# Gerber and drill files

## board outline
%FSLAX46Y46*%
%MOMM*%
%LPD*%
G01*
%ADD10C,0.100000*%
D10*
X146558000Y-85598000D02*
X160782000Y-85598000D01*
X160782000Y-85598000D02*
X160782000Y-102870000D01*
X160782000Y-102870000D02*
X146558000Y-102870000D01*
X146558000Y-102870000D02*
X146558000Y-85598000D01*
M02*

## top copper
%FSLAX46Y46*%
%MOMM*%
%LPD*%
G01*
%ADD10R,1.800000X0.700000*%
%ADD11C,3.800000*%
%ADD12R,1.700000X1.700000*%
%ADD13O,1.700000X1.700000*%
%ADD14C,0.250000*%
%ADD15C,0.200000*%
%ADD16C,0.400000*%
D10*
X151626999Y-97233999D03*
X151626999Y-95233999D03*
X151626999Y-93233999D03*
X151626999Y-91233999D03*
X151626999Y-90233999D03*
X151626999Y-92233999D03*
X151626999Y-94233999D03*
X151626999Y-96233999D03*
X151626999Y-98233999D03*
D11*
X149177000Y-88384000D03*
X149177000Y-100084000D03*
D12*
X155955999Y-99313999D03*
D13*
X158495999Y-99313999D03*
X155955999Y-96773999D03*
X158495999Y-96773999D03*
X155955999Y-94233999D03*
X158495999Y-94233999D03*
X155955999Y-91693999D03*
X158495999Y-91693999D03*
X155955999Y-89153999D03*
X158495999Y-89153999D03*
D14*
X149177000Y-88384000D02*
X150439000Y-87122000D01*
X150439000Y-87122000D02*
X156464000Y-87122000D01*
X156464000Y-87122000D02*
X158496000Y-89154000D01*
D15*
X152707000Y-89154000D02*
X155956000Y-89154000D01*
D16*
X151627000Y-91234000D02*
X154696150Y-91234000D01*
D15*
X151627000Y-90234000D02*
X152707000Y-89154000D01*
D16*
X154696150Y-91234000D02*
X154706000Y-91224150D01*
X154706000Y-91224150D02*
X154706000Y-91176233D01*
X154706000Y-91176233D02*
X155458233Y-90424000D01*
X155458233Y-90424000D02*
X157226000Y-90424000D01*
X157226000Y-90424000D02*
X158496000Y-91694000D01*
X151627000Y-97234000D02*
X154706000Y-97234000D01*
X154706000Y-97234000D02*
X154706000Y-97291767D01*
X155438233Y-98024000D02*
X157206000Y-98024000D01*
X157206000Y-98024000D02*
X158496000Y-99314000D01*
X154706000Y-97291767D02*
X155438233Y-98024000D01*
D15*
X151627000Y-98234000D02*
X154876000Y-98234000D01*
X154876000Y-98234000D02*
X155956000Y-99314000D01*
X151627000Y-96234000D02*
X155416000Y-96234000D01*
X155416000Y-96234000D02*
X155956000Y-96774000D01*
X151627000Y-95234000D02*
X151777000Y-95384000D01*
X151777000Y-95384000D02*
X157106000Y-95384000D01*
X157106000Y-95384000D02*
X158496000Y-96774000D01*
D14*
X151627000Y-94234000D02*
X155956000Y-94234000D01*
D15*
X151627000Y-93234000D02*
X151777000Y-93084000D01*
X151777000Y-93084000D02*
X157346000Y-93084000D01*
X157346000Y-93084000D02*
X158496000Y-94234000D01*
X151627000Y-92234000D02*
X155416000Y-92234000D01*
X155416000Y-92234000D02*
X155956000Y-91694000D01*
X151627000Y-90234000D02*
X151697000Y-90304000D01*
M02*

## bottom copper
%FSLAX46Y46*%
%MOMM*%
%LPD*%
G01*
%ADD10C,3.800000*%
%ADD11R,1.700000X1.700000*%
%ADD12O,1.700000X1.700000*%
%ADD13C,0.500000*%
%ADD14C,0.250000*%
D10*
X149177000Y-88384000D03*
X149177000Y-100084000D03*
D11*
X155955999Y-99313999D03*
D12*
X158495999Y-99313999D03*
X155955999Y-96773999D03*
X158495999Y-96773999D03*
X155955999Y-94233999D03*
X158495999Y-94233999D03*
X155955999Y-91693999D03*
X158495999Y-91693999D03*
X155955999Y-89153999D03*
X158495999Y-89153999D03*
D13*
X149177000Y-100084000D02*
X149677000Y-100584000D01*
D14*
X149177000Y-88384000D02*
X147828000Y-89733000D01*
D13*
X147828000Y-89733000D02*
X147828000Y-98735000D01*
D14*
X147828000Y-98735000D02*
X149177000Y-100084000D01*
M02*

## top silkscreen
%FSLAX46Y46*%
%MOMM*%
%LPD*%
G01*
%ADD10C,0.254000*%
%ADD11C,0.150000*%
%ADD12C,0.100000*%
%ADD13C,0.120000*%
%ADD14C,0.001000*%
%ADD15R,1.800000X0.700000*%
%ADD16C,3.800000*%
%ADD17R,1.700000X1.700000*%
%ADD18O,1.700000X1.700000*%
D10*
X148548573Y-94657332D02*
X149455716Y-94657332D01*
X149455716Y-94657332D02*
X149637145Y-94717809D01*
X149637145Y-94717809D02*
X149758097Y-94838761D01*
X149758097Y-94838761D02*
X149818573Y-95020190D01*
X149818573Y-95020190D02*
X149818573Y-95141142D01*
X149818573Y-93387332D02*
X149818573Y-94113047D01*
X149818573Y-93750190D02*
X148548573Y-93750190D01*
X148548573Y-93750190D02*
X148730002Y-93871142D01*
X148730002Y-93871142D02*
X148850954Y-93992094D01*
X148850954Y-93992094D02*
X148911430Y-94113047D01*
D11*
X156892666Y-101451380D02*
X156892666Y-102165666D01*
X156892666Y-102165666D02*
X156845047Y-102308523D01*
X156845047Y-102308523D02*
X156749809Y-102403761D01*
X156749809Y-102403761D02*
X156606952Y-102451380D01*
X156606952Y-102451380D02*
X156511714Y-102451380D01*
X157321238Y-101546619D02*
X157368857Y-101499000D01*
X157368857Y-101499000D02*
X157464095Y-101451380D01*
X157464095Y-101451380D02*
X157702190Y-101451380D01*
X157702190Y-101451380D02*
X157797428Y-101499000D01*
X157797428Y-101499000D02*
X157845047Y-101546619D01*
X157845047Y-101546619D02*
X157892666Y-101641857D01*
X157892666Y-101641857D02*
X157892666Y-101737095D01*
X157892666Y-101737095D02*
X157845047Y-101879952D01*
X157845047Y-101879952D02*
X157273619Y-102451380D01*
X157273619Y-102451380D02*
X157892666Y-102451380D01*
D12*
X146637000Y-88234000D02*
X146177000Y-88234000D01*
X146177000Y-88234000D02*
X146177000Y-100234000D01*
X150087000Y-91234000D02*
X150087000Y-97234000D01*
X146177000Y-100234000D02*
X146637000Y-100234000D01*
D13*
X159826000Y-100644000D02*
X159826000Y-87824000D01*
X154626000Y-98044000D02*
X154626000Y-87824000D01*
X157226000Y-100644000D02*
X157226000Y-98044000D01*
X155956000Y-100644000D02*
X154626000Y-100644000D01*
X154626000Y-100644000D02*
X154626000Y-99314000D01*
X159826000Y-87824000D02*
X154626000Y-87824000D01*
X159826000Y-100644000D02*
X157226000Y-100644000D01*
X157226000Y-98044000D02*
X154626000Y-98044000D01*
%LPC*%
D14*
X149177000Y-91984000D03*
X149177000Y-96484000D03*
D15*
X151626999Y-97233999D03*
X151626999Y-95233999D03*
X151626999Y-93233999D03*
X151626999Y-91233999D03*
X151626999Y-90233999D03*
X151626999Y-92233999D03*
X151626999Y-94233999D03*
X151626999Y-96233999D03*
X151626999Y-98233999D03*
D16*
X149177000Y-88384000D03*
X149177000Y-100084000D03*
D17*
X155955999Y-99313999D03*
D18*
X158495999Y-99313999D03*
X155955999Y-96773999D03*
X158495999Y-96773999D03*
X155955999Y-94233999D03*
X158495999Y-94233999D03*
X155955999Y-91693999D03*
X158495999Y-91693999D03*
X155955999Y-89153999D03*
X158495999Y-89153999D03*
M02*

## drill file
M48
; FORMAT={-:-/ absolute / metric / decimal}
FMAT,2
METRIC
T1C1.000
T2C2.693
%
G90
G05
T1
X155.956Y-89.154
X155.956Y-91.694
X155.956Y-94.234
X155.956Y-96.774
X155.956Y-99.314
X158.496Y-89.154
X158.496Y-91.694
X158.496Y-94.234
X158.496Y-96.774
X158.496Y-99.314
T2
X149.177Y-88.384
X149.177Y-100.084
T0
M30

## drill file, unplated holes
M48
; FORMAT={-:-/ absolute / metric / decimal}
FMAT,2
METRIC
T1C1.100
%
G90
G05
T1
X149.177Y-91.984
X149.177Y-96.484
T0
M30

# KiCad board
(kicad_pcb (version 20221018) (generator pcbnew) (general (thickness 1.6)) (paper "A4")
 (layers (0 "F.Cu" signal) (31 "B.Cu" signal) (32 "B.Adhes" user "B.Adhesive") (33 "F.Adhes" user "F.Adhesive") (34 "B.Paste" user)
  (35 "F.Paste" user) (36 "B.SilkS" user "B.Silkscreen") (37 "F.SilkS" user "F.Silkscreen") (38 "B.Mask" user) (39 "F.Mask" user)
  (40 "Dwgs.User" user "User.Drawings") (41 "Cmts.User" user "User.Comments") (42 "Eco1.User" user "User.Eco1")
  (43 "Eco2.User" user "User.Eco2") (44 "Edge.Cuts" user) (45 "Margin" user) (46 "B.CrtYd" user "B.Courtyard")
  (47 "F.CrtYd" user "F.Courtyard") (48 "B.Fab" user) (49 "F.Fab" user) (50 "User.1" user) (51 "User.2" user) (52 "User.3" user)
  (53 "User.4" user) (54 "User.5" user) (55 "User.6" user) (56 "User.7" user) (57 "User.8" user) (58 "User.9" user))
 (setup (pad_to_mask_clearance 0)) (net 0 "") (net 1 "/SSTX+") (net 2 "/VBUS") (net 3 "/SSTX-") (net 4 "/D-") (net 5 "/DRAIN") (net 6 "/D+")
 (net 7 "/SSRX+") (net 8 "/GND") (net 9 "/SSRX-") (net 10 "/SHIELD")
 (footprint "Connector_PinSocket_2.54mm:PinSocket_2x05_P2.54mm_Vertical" (layer "F.Cu") (at 155.956 99.314 180)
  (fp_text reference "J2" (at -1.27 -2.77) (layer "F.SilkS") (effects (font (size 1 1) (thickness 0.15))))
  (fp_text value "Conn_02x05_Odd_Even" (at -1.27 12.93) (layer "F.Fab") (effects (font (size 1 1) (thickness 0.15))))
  (fp_line (start -3.87 -1.33) (end -3.87 11.49) (stroke (width 0.12) (type solid)) (layer "F.SilkS"))
  (fp_line (start -3.87 -1.33) (end -1.27 -1.33) (stroke (width 0.12) (type solid)) (layer "F.SilkS"))
  (fp_line (start -3.87 11.49) (end 1.33 11.49) (stroke (width 0.12) (type solid)) (layer "F.SilkS"))
  (fp_line (start -1.27 -1.33) (end -1.27 1.27) (stroke (width 0.12) (type solid)) (layer "F.SilkS"))
  (fp_line (start -1.27 1.27) (end 1.33 1.27) (stroke (width 0.12) (type solid)) (layer "F.SilkS"))
  (fp_line (start 0 -1.33) (end 1.33 -1.33) (stroke (width 0.12) (type solid)) (layer "F.SilkS"))
  (fp_line (start 1.33 -1.33) (end 1.33 0) (stroke (width 0.12) (type solid)) (layer "F.SilkS"))
  (fp_line (start 1.33 1.27) (end 1.33 11.49) (stroke (width 0.12) (type solid)) (layer "F.SilkS"))
  (pad "1" thru_hole rect (at 0 0 180) (size 1.7 1.7) (drill 1) (layers "*.Cu" "*.Mask") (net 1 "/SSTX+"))
  (pad "2" thru_hole oval (at -2.54 0 180) (size 1.7 1.7) (drill 1) (layers "*.Cu" "*.Mask") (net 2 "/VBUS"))
  (pad "3" thru_hole oval (at 0 2.54 180) (size 1.7 1.7) (drill 1) (layers "*.Cu" "*.Mask") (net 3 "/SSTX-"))
  (pad "4" thru_hole oval (at -2.54 2.54 180) (size 1.7 1.7) (drill 1) (layers "*.Cu" "*.Mask") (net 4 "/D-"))
  (pad "5" thru_hole oval (at 0 5.08 180) (size 1.7 1.7) (drill 1) (layers "*.Cu" "*.Mask") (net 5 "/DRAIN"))
  (pad "6" thru_hole oval (at -2.54 5.08 180) (size 1.7 1.7) (drill 1) (layers "*.Cu" "*.Mask") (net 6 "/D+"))
  (pad "7" thru_hole oval (at 0 7.62 180) (size 1.7 1.7) (drill 1) (layers "*.Cu" "*.Mask") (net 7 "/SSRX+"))
  (pad "8" thru_hole oval (at -2.54 7.62 180) (size 1.7 1.7) (drill 1) (layers "*.Cu" "*.Mask") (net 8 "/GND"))
  (pad "9" thru_hole oval (at 0 10.16 180) (size 1.7 1.7) (drill 1) (layers "*.Cu" "*.Mask") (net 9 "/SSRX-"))
  (pad "10" thru_hole oval (at -2.54 10.16 180) (size 1.7 1.7) (drill 1) (layers "*.Cu" "*.Mask") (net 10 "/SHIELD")))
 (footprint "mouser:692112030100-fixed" (layer "F.Cu") (at 149.352 94.234 -90)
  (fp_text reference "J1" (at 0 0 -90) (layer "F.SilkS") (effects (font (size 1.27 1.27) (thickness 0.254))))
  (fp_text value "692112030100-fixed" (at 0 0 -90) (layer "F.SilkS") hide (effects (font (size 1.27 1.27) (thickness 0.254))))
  (fp_line (start -6 2.715) (end -6 3.175) (stroke (width 0.1) (type solid)) (layer "F.SilkS"))
  (fp_line (start -6 3.175) (end 6 3.175) (stroke (width 0.1) (type solid)) (layer "F.SilkS"))
  (fp_line (start -3 -0.735) (end 3 -0.735) (stroke (width 0.1) (type solid)) (layer "F.SilkS"))
  (fp_line (start 6 3.175) (end 6 2.715) (stroke (width 0.1) (type solid)) (layer "F.SilkS"))
  (pad "" np_thru_hole circle (at -2.25 0.175 270) (size 0.001 0.001) (drill 1.1) (layers "*.Cu" "*.Mask"))
  (pad "" np_thru_hole circle (at 2.25 0.175 270) (size 0.001 0.001) (drill 1.1) (layers "*.Cu" "*.Mask"))
  (pad "1" smd rect (at 3 -2.275 270) (size 0.7 1.8) (layers "F.Cu" "F.Paste" "F.Mask") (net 2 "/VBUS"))
  (pad "2" smd rect (at 1 -2.275 270) (size 0.7 1.8) (layers "F.Cu" "F.Paste" "F.Mask") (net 4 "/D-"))
  (pad "3" smd rect (at -1 -2.275 270) (size 0.7 1.8) (layers "F.Cu" "F.Paste" "F.Mask") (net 6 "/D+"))
  (pad "4" smd rect (at -3 -2.275 270) (size 0.7 1.8) (layers "F.Cu" "F.Paste" "F.Mask") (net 8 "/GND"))
  (pad "5" smd rect (at -4 -2.275 270) (size 0.7 1.8) (layers "F.Cu" "F.Paste" "F.Mask") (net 9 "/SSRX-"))
  (pad "6" smd rect (at -2 -2.275 270) (size 0.7 1.8) (layers "F.Cu" "F.Paste" "F.Mask") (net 7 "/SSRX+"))
  (pad "7" smd rect (at 0 -2.275 270) (size 0.7 1.8) (layers "F.Cu" "F.Paste" "F.Mask") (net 5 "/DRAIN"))
  (pad "8" smd rect (at 2 -2.275 270) (size 0.7 1.8) (layers "F.Cu" "F.Paste" "F.Mask") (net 3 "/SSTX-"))
  (pad "9" smd rect (at 4 -2.275 270) (size 0.7 1.8) (layers "F.Cu" "F.Paste" "F.Mask") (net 1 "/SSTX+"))
  (pad "10" thru_hole circle (at -5.85 0.175 270) (size 3.8 3.8) (drill 2.6926) (layers "*.Cu" "*.Mask") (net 10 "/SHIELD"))
  (pad "11" thru_hole circle (at 5.85 0.175 270) (size 3.8 3.8) (drill 2.6926) (layers "*.Cu" "*.Mask") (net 10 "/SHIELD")))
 (gr_rect (start 146.558 85.598) (end 160.782 102.87) (stroke (width 0.1) (type solid)) (fill none) (layer "Edge.Cuts"))
 (segment (start 155.438233 98.024) (end 157.206 98.024) (width 0.4) (layer "F.Cu") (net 2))
 (segment (start 154.706 97.291767) (end 155.438233 98.024) (width 0.4) (layer "F.Cu") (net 2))
 (segment (start 154.706 97.234) (end 154.706 97.291767) (width 0.4) (layer "F.Cu") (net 2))
 (segment (start 151.627 97.234) (end 154.706 97.234) (width 0.4) (layer "F.Cu") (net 2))
 (segment (start 157.206 98.024) (end 158.496 99.314) (width 0.4) (layer "F.Cu") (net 2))
 (segment (start 157.106 95.384) (end 158.496 96.774) (width 0.2) (layer "F.Cu") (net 4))
 (segment (start 151.627 95.234) (end 151.777 95.384) (width 0.2) (layer "F.Cu") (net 4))
 (segment (start 151.777 95.384) (end 157.106 95.384) (width 0.2) (layer "F.Cu") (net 4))
 (segment (start 151.777 93.084) (end 157.346 93.084) (width 0.2) (layer "F.Cu") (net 6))
 (segment (start 157.346 93.084) (end 158.496 94.234) (width 0.2) (layer "F.Cu") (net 6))
 (segment (start 151.627 93.234) (end 151.777 93.084) (width 0.2) (layer "F.Cu") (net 6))
 (segment (start 154.69615 91.234) (end 154.706 91.22415) (width 0.4) (layer "F.Cu") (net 8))
 (segment (start 154.706 91.176233) (end 155.458233 90.424) (width 0.4) (layer "F.Cu") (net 8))
 (segment (start 154.706 91.22415) (end 154.706 91.176233) (width 0.4) (layer "F.Cu") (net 8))
 (segment (start 157.226 90.424) (end 158.496 91.694) (width 0.4) (layer "F.Cu") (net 8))
 (segment (start 151.627 91.234) (end 154.69615 91.234) (width 0.4) (layer "F.Cu") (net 8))
 (segment (start 155.458233 90.424) (end 157.226 90.424) (width 0.4) (layer "F.Cu") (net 8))
 (segment (start 151.627 90.234) (end 151.697 90.304) (width 0.2) (layer "F.Cu") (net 9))
 (segment (start 152.707 89.154) (end 155.956 89.154) (width 0.2) (layer "F.Cu") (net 9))
 (segment (start 151.627 90.234) (end 152.707 89.154) (width 0.2) (layer "F.Cu") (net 9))
 (segment (start 151.627 92.234) (end 155.416 92.234) (width 0.2) (layer "F.Cu") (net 7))
 (segment (start 155.416 92.234) (end 155.956 91.694) (width 0.2) (layer "F.Cu") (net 7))
 (segment (start 151.627 94.234) (end 155.956 94.234) (width 0.25) (layer "F.Cu") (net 5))
 (segment (start 151.627 96.234) (end 155.416 96.234) (width 0.2) (layer "F.Cu") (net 3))
 (segment (start 155.416 96.234) (end 155.956 96.774) (width 0.2) (layer "F.Cu") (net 3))
 (segment (start 154.876 98.234) (end 155.956 99.314) (width 0.2) (layer "F.Cu") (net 1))
 (segment (start 151.627 98.234) (end 154.876 98.234) (width 0.2) (layer "F.Cu") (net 1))
 (segment (start 156.464 87.122) (end 158.496 89.154) (width 0.25) (layer "F.Cu") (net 10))
 (segment (start 150.439 87.122) (end 156.464 87.122) (width 0.25) (layer "F.Cu") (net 10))
 (segment (start 149.177 88.384) (end 150.439 87.122) (width 0.25) (layer "F.Cu") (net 10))
 (segment (start 149.177 100.084) (end 149.677 100.584) (width 0.5) (layer "B.Cu") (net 10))
 (segment (start 149.177 88.384) (end 147.828 89.733) (width 0.25) (layer "B.Cu") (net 10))
 (segment (start 147.828 98.735) (end 149.177 100.084) (width 0.25) (layer "B.Cu") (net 10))
 (segment (start 147.828 89.733) (end 147.828 98.735) (width 0.5) (layer "B.Cu") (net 10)))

